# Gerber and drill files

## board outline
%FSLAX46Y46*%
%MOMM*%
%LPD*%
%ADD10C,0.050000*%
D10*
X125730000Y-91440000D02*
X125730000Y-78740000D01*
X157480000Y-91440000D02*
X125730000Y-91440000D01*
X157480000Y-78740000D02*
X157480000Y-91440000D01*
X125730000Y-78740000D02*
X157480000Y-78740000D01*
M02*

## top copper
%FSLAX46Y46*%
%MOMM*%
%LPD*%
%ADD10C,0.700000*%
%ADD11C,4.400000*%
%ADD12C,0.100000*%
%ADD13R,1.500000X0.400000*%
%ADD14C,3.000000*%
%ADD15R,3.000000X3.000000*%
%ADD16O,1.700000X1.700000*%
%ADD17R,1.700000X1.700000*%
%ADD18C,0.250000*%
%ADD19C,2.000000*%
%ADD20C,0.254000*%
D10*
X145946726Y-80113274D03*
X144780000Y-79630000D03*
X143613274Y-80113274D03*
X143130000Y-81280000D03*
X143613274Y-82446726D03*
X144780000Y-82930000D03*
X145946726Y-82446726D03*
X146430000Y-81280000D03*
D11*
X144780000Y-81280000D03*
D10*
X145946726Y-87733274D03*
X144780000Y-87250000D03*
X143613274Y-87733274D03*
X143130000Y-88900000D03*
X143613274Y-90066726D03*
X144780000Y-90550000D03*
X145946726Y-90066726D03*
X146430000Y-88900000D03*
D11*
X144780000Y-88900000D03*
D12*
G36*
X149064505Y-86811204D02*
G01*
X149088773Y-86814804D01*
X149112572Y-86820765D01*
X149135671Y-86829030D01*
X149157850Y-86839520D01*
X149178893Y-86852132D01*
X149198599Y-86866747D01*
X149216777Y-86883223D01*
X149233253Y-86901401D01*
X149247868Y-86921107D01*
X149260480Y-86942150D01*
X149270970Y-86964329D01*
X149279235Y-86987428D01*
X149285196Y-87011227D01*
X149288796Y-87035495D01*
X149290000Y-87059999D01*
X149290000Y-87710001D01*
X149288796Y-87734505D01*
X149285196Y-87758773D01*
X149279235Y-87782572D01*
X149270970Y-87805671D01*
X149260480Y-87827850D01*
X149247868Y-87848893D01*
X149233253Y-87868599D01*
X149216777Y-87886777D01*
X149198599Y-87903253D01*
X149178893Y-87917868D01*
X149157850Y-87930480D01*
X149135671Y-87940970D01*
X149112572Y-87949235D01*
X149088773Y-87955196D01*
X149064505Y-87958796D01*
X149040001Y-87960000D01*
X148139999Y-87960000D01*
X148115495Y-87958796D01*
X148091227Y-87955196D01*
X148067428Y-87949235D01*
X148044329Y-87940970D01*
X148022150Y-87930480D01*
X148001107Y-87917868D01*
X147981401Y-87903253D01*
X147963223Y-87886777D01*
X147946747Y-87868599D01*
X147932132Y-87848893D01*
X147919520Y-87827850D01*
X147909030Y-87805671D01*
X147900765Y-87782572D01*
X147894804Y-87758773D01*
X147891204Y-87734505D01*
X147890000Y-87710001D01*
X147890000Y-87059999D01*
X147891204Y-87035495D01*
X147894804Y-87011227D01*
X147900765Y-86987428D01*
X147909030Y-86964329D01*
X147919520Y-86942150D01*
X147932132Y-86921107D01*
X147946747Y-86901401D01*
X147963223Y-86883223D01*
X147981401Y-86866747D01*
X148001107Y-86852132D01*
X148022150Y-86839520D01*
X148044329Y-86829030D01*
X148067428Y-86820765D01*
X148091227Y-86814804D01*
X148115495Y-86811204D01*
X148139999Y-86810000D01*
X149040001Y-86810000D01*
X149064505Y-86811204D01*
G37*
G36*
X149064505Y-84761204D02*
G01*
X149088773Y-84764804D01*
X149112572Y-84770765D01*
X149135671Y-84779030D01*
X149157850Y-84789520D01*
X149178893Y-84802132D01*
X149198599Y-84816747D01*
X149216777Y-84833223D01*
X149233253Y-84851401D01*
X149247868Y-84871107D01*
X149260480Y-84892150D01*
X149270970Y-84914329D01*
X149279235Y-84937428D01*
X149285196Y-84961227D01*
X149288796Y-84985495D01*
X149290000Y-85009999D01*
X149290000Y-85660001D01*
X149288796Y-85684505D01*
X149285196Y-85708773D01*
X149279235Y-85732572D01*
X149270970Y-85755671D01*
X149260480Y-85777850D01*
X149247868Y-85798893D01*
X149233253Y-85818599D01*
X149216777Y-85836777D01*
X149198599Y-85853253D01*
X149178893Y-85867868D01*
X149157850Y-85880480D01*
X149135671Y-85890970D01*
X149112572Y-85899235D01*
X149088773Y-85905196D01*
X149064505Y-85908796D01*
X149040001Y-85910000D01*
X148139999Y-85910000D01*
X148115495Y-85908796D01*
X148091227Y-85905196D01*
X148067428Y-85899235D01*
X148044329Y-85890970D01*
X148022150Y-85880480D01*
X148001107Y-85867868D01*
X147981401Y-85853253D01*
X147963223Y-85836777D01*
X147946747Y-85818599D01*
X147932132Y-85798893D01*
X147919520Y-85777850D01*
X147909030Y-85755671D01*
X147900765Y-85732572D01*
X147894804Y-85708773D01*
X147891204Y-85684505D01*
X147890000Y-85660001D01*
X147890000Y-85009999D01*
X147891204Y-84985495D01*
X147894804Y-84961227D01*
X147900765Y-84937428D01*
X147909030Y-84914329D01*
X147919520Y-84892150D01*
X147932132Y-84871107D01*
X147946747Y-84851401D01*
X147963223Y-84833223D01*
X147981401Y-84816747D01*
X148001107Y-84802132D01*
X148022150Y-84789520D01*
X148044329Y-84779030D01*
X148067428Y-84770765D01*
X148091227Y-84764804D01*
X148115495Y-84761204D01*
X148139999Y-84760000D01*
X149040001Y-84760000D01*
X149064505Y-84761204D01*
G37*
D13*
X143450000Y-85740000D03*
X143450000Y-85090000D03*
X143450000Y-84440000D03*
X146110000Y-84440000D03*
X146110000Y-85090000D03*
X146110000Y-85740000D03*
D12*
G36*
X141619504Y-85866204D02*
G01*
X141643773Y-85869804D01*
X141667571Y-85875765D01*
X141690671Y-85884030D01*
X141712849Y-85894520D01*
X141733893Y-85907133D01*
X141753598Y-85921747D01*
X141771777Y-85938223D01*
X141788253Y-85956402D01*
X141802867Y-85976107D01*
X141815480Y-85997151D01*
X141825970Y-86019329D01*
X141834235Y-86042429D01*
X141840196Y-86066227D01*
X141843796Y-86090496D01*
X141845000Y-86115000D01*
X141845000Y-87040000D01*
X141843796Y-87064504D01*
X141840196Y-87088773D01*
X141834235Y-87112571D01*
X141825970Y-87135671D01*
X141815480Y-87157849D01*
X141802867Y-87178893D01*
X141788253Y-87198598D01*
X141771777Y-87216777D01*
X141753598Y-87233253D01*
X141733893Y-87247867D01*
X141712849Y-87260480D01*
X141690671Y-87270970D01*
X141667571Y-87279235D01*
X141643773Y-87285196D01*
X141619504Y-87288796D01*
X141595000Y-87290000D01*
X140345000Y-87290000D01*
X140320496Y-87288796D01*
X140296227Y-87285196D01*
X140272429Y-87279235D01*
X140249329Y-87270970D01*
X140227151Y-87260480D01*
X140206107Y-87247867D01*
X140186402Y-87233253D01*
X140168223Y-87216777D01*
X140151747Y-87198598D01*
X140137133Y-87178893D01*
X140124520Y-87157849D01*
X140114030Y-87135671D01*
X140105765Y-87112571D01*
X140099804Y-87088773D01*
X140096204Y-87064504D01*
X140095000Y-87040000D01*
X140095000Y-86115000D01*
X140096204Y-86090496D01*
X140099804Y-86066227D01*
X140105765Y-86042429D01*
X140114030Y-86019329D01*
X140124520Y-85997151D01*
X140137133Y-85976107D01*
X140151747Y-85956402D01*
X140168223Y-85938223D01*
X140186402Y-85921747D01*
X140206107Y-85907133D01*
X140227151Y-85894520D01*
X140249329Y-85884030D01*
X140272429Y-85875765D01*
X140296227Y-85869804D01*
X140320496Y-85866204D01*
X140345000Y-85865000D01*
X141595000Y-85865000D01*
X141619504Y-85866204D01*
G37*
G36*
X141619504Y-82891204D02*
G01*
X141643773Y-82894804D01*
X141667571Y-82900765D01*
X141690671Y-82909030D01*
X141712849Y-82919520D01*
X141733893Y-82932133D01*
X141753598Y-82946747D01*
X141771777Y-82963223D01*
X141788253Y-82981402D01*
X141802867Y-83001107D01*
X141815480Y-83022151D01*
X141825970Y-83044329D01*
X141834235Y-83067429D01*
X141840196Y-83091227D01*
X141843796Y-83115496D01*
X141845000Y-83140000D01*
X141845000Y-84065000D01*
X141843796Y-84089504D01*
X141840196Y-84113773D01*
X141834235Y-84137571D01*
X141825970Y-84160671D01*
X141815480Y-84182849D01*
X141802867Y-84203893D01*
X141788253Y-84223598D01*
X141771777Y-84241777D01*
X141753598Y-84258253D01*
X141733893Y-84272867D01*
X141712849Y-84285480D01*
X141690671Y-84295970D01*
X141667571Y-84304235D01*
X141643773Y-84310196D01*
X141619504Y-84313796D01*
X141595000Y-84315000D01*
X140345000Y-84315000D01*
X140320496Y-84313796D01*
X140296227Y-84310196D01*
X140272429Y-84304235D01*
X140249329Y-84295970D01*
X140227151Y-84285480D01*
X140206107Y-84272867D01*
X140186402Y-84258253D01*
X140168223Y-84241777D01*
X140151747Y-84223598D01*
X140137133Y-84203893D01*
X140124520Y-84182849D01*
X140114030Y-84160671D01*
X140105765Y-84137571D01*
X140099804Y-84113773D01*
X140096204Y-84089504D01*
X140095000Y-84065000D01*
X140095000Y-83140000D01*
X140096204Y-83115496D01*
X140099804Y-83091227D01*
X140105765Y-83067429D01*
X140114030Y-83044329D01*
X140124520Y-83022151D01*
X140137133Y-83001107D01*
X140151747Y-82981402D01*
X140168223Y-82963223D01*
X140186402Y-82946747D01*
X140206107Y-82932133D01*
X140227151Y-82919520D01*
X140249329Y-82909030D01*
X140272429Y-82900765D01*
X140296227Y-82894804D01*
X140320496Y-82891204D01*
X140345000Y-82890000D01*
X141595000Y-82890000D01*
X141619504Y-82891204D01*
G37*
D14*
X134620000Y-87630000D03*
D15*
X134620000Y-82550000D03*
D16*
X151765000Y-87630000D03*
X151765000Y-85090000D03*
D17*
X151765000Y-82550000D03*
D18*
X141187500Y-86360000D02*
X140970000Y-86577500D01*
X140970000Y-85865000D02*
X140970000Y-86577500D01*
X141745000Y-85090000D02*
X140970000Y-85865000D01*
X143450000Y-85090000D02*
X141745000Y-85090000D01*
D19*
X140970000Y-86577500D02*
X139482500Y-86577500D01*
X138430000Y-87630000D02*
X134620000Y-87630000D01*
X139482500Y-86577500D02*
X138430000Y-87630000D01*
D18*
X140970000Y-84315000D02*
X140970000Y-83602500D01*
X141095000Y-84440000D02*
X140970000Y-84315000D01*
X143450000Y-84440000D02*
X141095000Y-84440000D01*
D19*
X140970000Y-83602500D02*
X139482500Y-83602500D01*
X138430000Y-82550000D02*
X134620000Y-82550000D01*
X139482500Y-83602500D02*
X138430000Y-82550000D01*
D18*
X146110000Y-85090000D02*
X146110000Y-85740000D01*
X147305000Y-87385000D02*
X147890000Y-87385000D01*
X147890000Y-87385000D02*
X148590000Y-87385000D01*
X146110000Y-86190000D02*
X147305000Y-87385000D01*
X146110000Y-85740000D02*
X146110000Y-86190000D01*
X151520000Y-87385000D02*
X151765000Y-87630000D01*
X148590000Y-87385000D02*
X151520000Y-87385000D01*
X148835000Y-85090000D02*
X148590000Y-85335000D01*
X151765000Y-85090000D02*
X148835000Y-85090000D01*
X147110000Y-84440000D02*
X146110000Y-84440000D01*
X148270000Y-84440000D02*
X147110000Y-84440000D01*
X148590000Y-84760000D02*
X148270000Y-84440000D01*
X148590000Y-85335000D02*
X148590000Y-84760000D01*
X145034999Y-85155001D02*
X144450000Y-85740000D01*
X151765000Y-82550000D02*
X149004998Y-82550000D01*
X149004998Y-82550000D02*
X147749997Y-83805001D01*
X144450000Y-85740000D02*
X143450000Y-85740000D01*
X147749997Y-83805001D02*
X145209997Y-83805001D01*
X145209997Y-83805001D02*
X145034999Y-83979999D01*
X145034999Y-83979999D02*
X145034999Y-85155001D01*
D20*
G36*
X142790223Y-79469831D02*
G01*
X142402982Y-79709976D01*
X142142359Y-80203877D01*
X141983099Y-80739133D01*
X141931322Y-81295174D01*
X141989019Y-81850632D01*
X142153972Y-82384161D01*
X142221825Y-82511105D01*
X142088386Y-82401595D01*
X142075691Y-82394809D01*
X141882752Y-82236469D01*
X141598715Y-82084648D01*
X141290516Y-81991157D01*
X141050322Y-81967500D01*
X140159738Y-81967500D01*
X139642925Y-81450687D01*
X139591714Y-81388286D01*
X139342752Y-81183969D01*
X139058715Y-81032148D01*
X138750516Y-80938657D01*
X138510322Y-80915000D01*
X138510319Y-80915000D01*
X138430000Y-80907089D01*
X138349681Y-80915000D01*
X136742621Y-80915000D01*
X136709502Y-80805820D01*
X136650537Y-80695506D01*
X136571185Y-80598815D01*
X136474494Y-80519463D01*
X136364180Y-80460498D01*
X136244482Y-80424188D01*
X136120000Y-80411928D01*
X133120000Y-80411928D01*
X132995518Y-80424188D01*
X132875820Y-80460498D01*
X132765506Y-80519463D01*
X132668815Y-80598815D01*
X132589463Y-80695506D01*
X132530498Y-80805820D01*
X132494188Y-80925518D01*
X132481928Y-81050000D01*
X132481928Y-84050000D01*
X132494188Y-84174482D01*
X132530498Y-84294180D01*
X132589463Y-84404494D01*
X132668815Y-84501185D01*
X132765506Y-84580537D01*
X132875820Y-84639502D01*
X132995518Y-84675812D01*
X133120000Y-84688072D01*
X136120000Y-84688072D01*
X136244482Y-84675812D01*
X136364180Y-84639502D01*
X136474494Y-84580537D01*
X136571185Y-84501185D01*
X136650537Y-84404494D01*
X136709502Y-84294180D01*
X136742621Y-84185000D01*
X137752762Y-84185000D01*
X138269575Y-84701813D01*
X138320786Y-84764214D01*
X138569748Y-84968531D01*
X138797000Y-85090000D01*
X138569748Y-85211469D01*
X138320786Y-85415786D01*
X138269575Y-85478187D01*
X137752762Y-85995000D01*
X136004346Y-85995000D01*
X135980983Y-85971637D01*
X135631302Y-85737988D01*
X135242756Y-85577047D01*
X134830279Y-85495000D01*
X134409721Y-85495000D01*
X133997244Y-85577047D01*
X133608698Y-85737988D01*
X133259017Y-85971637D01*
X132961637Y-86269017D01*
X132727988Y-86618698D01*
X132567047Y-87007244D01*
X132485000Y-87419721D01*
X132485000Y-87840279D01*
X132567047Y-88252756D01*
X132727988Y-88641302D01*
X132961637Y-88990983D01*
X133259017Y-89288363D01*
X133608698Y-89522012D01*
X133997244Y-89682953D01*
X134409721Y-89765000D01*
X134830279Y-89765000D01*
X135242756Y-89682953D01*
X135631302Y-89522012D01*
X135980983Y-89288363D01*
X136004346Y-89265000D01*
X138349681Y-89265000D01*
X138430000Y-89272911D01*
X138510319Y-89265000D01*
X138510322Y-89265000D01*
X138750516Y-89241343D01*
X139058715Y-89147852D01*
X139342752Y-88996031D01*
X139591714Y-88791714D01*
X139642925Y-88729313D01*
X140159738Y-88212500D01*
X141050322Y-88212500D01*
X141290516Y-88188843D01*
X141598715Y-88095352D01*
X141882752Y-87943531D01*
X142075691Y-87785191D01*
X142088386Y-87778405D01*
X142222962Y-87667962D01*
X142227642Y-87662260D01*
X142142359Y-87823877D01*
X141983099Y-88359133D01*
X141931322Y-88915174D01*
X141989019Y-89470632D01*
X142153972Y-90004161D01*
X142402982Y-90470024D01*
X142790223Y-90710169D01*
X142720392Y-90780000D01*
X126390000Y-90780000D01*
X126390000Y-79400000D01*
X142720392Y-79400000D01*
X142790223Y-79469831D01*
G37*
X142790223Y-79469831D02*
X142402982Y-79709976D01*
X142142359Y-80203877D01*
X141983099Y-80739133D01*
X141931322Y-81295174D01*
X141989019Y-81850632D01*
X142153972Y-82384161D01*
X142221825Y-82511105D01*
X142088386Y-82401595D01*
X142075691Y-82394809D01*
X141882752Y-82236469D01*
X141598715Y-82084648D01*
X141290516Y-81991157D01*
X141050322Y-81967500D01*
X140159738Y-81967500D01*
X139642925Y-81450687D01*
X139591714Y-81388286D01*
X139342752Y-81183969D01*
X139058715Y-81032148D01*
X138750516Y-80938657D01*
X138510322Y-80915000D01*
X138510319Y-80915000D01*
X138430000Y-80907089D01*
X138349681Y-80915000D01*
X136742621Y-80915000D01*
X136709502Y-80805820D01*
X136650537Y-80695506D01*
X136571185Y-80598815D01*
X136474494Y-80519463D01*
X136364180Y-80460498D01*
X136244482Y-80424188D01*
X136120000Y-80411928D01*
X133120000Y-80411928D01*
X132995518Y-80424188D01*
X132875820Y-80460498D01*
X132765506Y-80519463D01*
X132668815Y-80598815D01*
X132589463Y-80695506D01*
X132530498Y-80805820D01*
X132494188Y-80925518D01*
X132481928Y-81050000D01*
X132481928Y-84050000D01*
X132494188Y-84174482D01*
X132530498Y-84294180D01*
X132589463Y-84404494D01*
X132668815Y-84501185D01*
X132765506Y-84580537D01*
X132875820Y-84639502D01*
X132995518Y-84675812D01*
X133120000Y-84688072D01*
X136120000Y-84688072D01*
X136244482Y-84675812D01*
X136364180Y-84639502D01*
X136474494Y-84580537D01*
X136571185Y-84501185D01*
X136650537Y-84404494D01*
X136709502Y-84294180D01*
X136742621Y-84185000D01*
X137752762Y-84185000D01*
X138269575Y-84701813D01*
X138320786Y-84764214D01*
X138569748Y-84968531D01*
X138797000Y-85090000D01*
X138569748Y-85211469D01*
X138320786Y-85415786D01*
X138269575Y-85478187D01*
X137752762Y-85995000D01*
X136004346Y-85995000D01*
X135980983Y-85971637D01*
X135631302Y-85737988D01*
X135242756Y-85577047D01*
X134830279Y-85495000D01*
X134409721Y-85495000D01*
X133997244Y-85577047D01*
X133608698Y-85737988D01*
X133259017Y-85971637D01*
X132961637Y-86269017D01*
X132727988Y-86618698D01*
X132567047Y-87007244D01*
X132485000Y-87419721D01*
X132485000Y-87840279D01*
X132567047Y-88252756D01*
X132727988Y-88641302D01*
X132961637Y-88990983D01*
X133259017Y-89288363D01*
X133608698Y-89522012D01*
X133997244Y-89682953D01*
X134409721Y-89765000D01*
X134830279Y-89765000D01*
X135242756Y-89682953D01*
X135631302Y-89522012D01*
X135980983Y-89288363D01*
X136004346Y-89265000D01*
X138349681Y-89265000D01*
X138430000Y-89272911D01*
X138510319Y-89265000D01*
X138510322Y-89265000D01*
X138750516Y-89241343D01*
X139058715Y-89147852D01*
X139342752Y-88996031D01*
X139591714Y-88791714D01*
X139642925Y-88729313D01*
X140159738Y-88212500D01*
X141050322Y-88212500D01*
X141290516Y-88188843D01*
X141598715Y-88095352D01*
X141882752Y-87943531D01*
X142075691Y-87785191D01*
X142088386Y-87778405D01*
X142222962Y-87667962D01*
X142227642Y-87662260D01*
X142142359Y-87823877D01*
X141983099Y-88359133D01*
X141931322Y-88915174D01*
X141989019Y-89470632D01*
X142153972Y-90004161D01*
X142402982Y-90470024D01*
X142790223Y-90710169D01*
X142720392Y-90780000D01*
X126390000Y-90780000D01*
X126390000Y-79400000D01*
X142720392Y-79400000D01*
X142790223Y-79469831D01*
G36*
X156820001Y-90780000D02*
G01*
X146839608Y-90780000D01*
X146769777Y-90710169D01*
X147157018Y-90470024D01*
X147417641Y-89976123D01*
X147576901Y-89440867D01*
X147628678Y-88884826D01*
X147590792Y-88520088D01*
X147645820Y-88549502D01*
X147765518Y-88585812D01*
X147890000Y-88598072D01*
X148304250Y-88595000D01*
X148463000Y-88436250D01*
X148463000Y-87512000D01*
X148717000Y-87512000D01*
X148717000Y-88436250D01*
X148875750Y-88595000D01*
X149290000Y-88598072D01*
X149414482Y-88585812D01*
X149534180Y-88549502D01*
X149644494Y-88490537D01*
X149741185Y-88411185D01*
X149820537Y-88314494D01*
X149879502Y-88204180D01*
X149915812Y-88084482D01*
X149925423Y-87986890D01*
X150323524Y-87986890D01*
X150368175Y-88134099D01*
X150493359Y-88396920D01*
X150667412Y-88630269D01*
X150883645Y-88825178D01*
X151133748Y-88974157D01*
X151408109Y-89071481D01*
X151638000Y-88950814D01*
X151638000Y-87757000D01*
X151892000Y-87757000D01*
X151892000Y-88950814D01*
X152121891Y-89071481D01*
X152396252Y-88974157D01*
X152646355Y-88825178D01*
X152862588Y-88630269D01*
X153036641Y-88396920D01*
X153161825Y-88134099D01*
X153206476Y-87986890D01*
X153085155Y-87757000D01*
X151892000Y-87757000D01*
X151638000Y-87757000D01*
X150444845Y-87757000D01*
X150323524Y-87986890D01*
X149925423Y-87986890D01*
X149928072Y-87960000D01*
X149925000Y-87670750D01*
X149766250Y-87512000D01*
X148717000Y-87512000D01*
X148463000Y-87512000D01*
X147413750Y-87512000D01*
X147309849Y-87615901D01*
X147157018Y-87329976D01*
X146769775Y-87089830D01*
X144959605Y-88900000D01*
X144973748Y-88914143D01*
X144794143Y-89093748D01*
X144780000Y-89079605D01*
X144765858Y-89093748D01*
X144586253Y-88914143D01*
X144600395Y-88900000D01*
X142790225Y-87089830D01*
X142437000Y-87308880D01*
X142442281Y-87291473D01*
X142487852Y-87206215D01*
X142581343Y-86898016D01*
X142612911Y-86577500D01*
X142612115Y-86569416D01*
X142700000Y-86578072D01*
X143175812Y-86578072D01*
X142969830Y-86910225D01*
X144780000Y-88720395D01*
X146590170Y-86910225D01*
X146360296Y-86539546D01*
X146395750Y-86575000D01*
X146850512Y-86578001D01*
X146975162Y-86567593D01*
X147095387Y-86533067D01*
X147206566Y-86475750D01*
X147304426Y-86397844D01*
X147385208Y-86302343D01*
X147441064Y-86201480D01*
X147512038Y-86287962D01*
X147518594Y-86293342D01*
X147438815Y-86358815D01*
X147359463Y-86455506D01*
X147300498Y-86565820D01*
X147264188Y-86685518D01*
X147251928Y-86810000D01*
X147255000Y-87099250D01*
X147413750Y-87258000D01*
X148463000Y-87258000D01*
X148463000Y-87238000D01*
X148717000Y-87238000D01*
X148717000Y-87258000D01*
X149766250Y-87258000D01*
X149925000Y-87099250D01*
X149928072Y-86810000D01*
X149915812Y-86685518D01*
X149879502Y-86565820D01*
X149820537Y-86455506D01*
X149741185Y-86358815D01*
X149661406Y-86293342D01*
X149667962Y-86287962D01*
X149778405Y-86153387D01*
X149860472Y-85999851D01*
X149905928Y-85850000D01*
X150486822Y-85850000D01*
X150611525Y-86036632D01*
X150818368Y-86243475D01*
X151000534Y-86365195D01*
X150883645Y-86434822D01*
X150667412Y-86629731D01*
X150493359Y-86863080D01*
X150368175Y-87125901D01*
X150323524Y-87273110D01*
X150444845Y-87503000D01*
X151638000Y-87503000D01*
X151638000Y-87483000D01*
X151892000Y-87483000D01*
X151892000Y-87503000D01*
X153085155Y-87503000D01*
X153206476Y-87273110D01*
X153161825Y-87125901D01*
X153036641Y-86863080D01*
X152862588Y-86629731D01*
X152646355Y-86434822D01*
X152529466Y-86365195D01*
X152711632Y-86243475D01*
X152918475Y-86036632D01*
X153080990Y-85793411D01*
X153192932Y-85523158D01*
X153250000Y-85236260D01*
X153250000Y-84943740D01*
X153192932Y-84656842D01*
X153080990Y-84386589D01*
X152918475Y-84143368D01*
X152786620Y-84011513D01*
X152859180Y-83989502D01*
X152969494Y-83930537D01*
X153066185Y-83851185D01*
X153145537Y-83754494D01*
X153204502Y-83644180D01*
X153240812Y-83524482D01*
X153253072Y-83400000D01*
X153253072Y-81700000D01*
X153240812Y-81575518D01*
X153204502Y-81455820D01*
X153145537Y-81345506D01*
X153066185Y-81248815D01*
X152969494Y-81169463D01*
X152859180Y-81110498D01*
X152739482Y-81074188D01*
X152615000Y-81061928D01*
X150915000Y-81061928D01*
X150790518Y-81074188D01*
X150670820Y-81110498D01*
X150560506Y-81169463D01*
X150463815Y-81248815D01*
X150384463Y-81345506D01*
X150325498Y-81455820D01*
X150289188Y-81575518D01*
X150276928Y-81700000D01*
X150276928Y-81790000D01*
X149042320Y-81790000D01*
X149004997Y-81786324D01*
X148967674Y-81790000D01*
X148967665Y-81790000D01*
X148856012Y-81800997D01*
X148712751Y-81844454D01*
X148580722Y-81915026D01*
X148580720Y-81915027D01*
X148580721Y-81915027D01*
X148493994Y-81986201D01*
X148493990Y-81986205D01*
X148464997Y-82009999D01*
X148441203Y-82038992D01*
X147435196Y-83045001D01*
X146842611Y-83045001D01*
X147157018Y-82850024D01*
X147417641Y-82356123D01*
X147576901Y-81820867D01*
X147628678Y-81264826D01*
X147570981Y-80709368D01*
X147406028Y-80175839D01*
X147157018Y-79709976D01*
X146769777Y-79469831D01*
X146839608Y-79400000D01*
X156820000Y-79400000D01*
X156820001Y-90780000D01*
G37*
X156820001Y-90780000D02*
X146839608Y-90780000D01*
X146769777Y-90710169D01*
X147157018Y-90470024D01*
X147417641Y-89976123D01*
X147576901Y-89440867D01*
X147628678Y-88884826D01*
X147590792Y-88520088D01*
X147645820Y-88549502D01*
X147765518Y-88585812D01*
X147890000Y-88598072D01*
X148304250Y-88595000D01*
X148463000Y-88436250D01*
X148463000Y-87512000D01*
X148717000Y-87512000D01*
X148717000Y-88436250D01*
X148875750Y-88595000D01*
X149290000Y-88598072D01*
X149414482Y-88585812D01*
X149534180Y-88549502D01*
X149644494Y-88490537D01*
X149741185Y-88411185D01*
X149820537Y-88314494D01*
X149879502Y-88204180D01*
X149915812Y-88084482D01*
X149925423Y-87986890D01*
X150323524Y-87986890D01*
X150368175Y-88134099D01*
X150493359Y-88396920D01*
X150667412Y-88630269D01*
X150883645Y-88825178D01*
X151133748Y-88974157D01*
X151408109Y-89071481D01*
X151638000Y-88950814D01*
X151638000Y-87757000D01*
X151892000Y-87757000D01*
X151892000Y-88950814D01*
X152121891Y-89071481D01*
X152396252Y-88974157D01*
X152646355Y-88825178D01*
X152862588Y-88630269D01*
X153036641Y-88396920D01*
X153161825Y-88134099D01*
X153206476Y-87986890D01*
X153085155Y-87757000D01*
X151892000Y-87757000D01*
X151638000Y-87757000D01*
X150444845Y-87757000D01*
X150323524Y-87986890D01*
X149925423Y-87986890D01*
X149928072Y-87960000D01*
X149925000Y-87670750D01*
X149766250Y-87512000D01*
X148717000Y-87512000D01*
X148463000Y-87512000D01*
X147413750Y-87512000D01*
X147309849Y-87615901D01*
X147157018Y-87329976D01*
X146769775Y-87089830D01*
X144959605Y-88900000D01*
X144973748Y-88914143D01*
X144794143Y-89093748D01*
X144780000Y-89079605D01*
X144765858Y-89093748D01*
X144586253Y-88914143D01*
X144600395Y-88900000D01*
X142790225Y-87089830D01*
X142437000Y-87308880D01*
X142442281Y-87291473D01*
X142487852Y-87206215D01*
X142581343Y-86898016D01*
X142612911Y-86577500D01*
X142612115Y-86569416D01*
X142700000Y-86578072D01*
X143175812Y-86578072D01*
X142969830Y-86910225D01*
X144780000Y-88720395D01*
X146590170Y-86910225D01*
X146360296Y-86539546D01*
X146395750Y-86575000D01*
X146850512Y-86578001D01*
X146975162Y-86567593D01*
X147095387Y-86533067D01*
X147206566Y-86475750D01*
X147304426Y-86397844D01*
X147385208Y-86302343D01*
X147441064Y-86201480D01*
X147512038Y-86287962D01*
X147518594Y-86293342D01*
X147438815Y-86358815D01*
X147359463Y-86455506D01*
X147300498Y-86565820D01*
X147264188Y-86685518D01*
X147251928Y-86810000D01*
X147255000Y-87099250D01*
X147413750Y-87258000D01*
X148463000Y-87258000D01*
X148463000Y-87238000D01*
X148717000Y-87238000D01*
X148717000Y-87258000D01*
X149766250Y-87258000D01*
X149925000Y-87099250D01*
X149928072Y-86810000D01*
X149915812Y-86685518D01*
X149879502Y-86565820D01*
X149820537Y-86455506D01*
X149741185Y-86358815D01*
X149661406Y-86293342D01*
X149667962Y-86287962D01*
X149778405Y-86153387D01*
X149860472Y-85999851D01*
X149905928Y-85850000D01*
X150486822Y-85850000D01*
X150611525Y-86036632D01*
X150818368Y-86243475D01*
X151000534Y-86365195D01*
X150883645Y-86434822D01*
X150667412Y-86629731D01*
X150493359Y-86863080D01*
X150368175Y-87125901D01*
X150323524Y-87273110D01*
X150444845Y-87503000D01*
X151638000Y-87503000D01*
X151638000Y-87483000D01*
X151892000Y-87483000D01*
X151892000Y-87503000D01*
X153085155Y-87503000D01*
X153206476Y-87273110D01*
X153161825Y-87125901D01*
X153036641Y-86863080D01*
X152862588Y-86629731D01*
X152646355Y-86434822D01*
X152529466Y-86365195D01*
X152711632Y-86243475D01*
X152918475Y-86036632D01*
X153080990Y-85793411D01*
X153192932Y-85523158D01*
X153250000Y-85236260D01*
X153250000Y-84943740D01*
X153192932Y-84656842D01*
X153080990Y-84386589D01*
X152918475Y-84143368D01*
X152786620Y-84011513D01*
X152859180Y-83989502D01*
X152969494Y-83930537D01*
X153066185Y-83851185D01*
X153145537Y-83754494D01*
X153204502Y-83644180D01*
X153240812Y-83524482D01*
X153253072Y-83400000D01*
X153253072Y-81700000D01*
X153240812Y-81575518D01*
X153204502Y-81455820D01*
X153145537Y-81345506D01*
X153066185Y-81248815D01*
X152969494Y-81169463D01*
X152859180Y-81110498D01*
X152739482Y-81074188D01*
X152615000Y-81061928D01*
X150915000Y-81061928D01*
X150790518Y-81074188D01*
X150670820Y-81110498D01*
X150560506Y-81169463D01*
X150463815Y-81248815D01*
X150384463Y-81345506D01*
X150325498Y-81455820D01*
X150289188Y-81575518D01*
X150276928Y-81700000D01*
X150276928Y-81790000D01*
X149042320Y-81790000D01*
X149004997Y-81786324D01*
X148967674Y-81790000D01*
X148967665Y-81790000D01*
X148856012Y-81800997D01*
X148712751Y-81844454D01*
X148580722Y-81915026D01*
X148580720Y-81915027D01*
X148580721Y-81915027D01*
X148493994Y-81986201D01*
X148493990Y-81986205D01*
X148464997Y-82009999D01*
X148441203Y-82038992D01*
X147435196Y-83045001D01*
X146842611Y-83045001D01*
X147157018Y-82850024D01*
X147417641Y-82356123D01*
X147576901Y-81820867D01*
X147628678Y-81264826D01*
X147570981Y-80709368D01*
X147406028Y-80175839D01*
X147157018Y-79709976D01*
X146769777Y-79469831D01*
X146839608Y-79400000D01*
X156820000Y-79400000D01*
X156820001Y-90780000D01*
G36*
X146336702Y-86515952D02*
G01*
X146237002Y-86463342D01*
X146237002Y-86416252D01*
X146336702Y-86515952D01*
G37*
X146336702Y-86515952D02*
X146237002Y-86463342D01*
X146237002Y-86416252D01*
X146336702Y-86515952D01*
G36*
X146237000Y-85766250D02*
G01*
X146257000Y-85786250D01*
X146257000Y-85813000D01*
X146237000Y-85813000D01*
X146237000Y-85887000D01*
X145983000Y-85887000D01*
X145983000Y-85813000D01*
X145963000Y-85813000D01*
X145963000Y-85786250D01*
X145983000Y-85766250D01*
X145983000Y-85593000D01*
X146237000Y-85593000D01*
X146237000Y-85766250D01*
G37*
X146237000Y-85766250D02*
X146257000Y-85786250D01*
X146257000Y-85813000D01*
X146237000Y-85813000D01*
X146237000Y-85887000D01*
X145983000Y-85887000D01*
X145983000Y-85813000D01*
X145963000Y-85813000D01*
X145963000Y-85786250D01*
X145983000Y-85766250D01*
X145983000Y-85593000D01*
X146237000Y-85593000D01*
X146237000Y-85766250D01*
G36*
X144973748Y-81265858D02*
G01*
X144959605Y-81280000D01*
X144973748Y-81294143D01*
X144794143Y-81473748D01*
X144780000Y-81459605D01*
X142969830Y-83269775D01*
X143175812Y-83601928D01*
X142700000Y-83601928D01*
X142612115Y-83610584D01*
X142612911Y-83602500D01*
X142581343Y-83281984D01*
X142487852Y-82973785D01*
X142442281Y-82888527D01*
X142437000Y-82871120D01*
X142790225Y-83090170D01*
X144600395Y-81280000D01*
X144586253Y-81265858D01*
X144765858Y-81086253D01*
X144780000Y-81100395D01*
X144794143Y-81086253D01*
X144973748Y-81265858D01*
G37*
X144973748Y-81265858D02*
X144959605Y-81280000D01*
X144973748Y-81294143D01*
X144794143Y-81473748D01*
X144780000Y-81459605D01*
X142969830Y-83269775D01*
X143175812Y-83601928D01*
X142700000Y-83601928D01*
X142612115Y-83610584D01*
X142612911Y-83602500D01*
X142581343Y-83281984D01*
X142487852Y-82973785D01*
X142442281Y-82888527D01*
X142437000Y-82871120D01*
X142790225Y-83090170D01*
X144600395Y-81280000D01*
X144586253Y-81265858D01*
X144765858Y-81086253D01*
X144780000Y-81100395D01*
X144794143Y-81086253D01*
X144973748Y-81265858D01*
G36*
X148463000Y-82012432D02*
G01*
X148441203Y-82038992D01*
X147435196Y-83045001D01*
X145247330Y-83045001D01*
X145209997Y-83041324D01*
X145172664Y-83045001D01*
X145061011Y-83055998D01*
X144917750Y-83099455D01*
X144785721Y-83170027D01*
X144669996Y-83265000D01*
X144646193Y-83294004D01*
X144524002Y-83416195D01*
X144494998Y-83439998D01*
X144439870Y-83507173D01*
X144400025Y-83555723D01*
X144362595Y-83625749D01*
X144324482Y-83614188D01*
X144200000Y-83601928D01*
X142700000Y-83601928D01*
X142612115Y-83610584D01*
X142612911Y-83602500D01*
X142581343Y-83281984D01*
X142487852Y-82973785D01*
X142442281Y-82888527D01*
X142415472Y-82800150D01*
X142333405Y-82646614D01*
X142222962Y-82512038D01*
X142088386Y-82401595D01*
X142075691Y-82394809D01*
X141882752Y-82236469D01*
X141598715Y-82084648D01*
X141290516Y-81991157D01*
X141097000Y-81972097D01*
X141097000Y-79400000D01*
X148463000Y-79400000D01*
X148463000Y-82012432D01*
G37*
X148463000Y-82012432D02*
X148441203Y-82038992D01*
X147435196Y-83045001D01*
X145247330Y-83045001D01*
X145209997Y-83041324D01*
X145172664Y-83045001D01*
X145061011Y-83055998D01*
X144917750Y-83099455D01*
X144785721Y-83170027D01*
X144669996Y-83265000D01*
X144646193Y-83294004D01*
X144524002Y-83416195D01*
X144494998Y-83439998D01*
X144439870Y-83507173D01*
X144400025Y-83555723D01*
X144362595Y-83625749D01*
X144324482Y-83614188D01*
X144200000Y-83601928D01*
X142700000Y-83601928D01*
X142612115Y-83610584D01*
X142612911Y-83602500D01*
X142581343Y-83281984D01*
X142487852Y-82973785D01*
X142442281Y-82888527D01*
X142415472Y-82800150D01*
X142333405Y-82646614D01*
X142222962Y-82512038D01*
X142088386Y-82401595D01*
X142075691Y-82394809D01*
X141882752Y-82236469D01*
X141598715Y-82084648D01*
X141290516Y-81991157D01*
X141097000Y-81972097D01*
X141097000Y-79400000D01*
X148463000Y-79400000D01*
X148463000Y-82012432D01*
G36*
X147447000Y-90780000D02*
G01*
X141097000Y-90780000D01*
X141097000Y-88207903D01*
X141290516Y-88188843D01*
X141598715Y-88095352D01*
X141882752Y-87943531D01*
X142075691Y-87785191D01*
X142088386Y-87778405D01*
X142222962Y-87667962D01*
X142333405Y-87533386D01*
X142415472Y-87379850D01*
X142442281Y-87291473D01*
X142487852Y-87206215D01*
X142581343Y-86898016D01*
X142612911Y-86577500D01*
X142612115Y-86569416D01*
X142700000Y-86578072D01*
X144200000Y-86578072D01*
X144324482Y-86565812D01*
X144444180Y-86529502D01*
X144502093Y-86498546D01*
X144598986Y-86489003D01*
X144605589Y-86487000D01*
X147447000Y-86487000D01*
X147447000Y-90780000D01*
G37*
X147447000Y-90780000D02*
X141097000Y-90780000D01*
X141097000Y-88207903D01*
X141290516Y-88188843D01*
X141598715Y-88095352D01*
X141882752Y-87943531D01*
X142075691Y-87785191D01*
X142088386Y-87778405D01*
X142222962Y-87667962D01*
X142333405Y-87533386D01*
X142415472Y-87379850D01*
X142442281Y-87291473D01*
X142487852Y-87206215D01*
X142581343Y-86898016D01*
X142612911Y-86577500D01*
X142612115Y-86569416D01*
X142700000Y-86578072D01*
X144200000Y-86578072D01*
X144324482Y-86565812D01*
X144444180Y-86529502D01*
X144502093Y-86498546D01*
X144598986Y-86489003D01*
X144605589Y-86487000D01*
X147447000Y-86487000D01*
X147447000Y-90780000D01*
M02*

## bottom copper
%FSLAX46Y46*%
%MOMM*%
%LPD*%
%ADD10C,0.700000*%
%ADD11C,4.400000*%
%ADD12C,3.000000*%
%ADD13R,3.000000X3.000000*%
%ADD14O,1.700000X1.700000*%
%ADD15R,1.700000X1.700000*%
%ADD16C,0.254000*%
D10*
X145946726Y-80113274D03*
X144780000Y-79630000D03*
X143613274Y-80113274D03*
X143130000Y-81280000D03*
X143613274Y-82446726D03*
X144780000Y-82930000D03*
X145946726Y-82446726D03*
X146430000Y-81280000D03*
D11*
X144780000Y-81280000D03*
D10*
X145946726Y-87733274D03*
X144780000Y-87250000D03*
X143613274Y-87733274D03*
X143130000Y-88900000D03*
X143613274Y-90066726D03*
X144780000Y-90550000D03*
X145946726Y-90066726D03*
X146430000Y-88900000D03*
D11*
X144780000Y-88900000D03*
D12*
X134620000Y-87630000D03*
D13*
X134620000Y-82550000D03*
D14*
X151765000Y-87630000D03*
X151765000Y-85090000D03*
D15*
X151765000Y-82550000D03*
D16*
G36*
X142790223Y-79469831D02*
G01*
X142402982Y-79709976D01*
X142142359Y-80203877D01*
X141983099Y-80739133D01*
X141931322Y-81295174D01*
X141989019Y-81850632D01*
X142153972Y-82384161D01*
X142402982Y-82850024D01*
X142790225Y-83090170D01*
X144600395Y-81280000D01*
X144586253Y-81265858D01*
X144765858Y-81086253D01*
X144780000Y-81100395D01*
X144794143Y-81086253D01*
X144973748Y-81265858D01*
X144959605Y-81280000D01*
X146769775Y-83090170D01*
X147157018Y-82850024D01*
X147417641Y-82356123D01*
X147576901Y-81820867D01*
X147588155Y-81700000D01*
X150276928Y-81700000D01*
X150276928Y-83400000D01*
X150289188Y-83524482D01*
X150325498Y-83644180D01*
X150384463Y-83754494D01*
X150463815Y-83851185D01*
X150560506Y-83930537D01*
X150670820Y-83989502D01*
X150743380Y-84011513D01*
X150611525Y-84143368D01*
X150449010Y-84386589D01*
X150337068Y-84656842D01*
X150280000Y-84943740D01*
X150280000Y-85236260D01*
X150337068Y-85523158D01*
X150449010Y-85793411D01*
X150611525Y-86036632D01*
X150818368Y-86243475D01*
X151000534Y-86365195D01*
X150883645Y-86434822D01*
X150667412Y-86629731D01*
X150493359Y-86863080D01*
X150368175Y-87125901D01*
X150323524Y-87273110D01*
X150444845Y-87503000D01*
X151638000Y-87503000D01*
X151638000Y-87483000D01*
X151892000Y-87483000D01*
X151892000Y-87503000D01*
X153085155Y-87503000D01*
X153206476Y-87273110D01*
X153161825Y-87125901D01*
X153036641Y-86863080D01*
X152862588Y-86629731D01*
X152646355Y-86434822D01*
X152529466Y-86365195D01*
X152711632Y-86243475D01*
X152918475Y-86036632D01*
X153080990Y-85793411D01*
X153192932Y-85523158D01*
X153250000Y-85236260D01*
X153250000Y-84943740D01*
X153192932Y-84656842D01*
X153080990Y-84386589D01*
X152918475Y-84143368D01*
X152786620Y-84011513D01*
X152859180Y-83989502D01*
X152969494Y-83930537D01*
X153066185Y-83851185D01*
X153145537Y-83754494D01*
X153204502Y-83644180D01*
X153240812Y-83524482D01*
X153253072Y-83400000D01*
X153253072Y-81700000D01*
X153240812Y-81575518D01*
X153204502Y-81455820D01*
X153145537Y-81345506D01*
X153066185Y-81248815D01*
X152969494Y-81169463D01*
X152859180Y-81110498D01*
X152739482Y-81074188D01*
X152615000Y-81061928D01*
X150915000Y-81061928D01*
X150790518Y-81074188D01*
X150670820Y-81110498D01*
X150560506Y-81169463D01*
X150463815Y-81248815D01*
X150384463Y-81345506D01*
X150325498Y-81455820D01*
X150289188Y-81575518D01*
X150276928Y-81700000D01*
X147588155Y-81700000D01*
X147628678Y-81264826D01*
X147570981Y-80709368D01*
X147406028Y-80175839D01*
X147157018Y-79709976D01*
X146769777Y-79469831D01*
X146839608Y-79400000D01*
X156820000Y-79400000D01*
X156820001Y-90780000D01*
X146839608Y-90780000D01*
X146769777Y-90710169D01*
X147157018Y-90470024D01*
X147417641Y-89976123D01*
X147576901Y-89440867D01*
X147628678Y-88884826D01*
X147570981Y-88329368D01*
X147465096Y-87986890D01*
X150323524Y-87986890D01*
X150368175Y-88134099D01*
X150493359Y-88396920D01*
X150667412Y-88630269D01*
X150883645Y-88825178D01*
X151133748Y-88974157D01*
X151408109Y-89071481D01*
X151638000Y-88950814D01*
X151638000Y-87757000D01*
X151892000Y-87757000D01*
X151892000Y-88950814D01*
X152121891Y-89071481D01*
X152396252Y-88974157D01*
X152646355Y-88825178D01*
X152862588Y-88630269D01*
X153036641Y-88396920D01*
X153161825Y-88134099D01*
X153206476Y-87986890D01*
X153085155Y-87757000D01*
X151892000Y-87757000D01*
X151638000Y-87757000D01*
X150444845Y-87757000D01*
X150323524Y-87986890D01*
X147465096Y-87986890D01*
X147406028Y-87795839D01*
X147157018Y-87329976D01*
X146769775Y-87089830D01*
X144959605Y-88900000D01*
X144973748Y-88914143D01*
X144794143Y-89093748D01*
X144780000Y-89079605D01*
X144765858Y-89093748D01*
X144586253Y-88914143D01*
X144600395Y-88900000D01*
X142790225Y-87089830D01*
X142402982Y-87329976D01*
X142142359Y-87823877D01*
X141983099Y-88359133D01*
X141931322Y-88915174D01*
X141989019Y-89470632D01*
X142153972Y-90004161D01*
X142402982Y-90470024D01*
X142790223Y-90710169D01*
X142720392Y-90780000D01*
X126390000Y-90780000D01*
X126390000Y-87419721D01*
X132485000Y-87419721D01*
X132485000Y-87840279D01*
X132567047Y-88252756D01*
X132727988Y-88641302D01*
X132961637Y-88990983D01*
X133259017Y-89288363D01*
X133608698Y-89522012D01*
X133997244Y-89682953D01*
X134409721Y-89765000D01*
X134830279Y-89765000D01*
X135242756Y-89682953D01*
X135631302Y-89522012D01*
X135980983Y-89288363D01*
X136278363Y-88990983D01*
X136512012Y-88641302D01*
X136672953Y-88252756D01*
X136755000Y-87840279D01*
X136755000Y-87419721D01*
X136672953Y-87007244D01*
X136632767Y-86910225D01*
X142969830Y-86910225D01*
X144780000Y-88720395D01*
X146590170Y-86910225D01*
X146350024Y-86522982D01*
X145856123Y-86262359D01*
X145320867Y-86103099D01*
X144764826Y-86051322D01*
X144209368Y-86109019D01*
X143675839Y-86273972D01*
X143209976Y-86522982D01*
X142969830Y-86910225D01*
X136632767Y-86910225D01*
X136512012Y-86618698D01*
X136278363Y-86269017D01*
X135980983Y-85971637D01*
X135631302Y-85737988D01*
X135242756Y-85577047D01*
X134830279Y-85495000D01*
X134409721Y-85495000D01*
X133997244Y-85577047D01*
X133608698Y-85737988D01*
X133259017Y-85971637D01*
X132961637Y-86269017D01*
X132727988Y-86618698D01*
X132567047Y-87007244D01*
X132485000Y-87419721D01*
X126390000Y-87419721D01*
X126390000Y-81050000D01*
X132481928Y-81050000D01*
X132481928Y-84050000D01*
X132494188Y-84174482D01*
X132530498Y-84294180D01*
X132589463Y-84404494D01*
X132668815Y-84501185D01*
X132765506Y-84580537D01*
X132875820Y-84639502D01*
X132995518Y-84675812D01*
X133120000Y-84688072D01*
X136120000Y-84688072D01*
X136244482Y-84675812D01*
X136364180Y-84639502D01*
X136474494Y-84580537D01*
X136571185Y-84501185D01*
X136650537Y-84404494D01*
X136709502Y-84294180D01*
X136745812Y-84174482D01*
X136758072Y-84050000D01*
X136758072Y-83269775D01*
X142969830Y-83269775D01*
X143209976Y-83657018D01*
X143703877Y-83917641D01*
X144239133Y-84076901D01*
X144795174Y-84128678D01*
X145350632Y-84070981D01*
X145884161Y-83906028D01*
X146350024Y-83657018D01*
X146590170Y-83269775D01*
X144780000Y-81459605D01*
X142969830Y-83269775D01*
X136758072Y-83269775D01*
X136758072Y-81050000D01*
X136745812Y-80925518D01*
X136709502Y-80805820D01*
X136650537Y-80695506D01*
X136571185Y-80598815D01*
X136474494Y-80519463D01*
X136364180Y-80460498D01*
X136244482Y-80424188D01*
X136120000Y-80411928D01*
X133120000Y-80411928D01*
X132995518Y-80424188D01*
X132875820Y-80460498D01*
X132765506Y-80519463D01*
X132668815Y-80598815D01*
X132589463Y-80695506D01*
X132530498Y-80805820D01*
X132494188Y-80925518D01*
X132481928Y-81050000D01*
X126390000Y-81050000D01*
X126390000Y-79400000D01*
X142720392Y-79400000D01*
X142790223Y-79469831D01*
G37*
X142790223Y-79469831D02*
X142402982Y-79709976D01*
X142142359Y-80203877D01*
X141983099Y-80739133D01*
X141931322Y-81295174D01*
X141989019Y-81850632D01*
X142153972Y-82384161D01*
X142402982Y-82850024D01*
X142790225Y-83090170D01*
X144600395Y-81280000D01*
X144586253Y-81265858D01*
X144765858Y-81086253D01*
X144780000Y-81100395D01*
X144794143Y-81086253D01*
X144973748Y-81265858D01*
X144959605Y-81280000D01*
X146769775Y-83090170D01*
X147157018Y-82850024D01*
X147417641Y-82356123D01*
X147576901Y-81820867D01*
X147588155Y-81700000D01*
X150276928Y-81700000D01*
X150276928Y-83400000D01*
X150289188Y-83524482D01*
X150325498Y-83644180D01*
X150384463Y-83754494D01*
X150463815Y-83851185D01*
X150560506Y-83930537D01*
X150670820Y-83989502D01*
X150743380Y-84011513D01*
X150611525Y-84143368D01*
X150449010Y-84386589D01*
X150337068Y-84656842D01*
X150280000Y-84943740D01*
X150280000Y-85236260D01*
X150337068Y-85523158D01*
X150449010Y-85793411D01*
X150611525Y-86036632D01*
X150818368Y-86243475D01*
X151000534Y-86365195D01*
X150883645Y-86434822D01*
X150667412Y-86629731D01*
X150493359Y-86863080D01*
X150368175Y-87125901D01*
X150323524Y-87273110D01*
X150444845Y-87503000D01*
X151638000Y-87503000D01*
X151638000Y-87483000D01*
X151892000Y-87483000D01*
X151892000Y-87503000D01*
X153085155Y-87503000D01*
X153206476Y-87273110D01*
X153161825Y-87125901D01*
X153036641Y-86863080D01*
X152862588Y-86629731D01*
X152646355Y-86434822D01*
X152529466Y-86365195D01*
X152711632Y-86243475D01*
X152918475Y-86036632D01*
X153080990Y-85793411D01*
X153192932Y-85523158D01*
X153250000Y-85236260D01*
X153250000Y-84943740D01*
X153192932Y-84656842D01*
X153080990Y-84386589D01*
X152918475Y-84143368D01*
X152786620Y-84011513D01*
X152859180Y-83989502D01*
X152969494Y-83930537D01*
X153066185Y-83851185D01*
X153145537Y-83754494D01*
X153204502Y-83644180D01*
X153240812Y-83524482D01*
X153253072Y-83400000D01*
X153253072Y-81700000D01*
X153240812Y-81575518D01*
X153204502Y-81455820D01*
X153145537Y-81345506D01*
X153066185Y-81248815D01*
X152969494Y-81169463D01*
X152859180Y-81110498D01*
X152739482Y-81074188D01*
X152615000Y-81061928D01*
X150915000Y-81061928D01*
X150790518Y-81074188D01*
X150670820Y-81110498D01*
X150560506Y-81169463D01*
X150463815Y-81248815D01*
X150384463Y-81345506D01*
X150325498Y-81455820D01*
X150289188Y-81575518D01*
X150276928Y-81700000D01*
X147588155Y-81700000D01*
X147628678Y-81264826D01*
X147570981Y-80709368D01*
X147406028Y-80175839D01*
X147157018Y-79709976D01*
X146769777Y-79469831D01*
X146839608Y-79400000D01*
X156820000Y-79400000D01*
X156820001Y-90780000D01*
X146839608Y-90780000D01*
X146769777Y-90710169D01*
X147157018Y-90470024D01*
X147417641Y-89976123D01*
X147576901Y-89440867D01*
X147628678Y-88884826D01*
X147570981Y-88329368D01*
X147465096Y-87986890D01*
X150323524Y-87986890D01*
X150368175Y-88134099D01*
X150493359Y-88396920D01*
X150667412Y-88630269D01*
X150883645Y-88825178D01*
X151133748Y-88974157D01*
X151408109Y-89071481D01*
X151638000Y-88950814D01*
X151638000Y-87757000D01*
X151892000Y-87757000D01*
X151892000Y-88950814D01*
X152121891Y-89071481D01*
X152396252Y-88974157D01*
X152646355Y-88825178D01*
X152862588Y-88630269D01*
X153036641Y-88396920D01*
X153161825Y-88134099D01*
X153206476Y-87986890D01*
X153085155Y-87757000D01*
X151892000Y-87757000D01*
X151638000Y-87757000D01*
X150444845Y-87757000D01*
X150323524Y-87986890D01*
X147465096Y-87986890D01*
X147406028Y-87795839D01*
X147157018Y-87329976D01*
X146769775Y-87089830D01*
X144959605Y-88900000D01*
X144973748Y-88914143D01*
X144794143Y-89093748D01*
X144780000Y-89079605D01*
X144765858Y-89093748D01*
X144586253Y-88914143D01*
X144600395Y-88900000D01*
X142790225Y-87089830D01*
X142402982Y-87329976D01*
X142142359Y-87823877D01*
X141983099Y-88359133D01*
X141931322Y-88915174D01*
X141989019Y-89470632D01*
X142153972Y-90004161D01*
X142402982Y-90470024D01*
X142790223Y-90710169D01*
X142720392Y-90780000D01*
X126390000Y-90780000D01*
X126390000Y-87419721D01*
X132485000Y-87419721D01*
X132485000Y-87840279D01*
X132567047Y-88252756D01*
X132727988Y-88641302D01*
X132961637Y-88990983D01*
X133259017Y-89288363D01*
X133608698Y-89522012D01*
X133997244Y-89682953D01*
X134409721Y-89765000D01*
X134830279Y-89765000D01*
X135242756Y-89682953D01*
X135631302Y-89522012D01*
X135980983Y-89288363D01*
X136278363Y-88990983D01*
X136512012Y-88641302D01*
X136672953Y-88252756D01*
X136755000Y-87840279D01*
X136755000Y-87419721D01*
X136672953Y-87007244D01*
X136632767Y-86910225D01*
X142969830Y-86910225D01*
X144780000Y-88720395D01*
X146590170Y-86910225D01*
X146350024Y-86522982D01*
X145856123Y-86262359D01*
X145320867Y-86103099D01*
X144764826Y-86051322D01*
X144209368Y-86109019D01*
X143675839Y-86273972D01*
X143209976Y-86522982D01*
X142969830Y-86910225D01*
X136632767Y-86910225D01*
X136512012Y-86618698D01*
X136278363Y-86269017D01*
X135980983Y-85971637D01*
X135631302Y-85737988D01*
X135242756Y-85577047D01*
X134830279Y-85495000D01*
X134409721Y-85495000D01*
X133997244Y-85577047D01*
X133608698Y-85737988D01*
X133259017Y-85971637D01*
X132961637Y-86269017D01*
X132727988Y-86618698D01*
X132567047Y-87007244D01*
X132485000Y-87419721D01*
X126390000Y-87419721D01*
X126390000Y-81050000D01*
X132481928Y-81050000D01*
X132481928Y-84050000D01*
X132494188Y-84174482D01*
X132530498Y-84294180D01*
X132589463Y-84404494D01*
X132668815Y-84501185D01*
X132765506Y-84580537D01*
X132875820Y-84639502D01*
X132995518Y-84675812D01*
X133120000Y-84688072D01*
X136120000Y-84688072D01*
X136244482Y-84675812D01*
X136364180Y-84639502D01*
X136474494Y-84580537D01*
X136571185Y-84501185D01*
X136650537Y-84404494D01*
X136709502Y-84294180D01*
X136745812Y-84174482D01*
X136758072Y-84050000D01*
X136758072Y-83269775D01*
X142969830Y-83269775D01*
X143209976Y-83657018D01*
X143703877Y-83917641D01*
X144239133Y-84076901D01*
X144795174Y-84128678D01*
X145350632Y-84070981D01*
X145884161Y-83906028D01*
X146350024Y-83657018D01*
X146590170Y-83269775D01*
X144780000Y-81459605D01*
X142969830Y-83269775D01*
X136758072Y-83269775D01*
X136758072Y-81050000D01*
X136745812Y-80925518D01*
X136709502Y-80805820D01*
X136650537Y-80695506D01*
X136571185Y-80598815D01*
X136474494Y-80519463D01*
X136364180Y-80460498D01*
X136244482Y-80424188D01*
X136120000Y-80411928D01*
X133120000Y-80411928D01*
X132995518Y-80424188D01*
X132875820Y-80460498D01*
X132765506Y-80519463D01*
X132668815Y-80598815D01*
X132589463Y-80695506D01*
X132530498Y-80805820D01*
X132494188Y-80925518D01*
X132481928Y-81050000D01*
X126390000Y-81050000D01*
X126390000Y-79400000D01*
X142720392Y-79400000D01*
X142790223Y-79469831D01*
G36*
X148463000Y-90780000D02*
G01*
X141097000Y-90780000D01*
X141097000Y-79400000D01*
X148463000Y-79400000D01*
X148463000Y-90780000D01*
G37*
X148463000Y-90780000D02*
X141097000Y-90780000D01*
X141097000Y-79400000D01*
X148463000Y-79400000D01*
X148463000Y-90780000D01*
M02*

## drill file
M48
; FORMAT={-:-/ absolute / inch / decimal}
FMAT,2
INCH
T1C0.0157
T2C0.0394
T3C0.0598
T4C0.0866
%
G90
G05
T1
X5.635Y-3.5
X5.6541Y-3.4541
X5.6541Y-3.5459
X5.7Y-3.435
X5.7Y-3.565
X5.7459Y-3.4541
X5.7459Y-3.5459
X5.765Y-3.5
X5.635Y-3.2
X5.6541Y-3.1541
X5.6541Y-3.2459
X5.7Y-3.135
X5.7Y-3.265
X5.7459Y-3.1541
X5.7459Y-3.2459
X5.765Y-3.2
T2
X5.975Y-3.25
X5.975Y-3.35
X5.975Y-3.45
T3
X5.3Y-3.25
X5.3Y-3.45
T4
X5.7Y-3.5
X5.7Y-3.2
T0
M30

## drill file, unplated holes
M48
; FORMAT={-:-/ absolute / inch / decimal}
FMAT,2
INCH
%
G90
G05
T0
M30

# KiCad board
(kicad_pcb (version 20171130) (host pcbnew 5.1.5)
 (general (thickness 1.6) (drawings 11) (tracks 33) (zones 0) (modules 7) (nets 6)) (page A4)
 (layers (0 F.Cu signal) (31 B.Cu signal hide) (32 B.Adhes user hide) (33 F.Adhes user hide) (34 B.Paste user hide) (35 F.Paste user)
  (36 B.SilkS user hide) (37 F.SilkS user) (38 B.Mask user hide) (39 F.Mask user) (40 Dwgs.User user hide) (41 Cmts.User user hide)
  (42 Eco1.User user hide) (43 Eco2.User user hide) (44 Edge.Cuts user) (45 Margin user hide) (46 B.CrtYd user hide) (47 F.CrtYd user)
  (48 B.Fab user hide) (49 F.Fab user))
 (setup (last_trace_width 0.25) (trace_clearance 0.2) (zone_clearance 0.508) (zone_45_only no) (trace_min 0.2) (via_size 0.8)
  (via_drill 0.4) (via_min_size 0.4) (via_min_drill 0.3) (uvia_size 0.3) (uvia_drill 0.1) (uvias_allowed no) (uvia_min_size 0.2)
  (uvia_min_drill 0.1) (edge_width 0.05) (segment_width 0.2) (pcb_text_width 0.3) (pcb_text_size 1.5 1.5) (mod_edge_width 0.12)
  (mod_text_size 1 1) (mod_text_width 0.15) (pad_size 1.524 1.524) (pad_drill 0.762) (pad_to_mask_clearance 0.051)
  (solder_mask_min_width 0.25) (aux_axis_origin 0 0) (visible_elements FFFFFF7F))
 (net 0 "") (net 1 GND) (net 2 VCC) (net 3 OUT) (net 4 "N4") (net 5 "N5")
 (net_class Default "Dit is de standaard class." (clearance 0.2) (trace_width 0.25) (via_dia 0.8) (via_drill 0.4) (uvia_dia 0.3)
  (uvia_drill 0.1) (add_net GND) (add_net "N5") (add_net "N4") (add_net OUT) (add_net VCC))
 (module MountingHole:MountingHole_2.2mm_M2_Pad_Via (layer F.Cu) (at 144.78 81.28)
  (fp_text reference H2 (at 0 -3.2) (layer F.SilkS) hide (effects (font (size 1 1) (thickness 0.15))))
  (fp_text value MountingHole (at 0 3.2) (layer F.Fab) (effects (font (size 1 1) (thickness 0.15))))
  (pad 1 thru_hole circle (at 1.166726 -1.166726) (size 0.7 0.7) (drill 0.4) (layers *.Cu *.Mask) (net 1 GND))
  (pad 1 thru_hole circle (at 0 -1.65) (size 0.7 0.7) (drill 0.4) (layers *.Cu *.Mask) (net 1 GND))
  (pad 1 thru_hole circle (at -1.166726 -1.166726) (size 0.7 0.7) (drill 0.4) (layers *.Cu *.Mask) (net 1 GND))
  (pad 1 thru_hole circle (at -1.65 0) (size 0.7 0.7) (drill 0.4) (layers *.Cu *.Mask) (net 1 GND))
  (pad 1 thru_hole circle (at -1.166726 1.166726) (size 0.7 0.7) (drill 0.4) (layers *.Cu *.Mask) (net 1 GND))
  (pad 1 thru_hole circle (at 0 1.65) (size 0.7 0.7) (drill 0.4) (layers *.Cu *.Mask) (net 1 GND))
  (pad 1 thru_hole circle (at 1.166726 1.166726) (size 0.7 0.7) (drill 0.4) (layers *.Cu *.Mask) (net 1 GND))
  (pad 1 thru_hole circle (at 1.65 0) (size 0.7 0.7) (drill 0.4) (layers *.Cu *.Mask) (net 1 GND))
  (pad 1 thru_hole circle (at 0 0) (size 4.4 4.4) (drill 2.2) (layers *.Cu *.Mask) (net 1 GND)))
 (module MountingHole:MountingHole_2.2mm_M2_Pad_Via (layer F.Cu) (at 144.78 88.9)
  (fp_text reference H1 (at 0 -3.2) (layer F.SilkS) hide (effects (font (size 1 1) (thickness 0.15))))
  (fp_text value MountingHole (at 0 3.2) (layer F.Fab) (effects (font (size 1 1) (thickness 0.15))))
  (pad 1 thru_hole circle (at 1.166726 -1.166726) (size 0.7 0.7) (drill 0.4) (layers *.Cu *.Mask) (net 1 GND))
  (pad 1 thru_hole circle (at 0 -1.65) (size 0.7 0.7) (drill 0.4) (layers *.Cu *.Mask) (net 1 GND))
  (pad 1 thru_hole circle (at -1.166726 -1.166726) (size 0.7 0.7) (drill 0.4) (layers *.Cu *.Mask) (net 1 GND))
  (pad 1 thru_hole circle (at -1.65 0) (size 0.7 0.7) (drill 0.4) (layers *.Cu *.Mask) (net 1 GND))
  (pad 1 thru_hole circle (at -1.166726 1.166726) (size 0.7 0.7) (drill 0.4) (layers *.Cu *.Mask) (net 1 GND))
  (pad 1 thru_hole circle (at 0 1.65) (size 0.7 0.7) (drill 0.4) (layers *.Cu *.Mask) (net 1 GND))
  (pad 1 thru_hole circle (at 1.166726 1.166726) (size 0.7 0.7) (drill 0.4) (layers *.Cu *.Mask) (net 1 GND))
  (pad 1 thru_hole circle (at 1.65 0) (size 0.7 0.7) (drill 0.4) (layers *.Cu *.Mask) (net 1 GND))
  (pad 1 thru_hole circle (at 0 0) (size 4.4 4.4) (drill 2.2) (layers *.Cu *.Mask) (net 1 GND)))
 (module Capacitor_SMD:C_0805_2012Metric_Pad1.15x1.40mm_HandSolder (layer F.Cu) (at 148.59 86.36 270)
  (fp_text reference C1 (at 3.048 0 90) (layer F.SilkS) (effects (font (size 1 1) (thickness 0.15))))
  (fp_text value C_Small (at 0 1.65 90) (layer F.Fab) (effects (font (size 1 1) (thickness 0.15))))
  (pad 2 smd roundrect (at 1.025 0 270) (size 1.15 1.4) (layers F.Cu F.Paste F.Mask) (roundrect_rratio 0.217391) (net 1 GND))
  (pad 1 smd roundrect (at -1.025 0 270) (size 1.15 1.4) (layers F.Cu F.Paste F.Mask) (roundrect_rratio 0.217391) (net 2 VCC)))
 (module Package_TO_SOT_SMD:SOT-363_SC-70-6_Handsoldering (layer F.Cu) (at 144.78 85.09 180)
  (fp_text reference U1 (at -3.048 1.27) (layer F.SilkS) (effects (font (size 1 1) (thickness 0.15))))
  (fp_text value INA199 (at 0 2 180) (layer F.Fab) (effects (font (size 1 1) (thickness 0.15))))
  (pad 6 smd rect (at 1.33 -0.65 180) (size 1.5 0.4) (layers F.Cu F.Paste F.Mask) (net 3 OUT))
  (pad 5 smd rect (at 1.33 0 180) (size 1.5 0.4) (layers F.Cu F.Paste F.Mask) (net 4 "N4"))
  (pad 4 smd rect (at 1.33 0.65 180) (size 1.5 0.4) (layers F.Cu F.Paste F.Mask) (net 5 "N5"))
  (pad 3 smd rect (at -1.33 0.65 180) (size 1.5 0.4) (layers F.Cu F.Paste F.Mask) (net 2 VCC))
  (pad 2 smd rect (at -1.33 0 180) (size 1.5 0.4) (layers F.Cu F.Paste F.Mask) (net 1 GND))
  (pad 1 smd rect (at -1.33 -0.65 180) (size 1.5 0.4) (layers F.Cu F.Paste F.Mask) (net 1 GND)))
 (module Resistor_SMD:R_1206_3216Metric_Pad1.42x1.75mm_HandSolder (layer F.Cu) (at 140.97 85.09 270)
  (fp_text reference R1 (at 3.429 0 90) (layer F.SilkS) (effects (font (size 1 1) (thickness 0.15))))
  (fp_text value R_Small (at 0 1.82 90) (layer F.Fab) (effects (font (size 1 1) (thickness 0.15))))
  (pad 2 smd roundrect (at 1.4875 0 270) (size 1.425 1.75) (layers F.Cu F.Paste F.Mask) (roundrect_rratio 0.175439) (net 4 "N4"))
  (pad 1 smd roundrect (at -1.4875 0 270) (size 1.425 1.75) (layers F.Cu F.Paste F.Mask) (roundrect_rratio 0.175439) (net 5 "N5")))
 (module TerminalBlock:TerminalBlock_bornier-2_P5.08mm (layer F.Cu) (at 134.62 82.55 270)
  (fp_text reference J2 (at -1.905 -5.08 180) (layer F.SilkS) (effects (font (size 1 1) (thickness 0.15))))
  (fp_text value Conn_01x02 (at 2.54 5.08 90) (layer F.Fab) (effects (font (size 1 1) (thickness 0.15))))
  (pad 2 thru_hole circle (at 5.08 0 270) (size 3 3) (drill 1.52) (layers *.Cu *.Mask) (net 4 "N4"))
  (pad 1 thru_hole rect (at 0 0 270) (size 3 3) (drill 1.52) (layers *.Cu *.Mask) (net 5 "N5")))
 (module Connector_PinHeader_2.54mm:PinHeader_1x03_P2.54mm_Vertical (layer F.Cu) (at 151.765 82.55)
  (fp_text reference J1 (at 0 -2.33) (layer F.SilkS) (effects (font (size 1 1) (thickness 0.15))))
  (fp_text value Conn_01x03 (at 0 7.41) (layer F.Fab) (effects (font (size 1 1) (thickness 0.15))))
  (pad 3 thru_hole oval (at 0 5.08) (size 1.7 1.7) (drill 1) (layers *.Cu *.Mask) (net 1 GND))
  (pad 2 thru_hole oval (at 0 2.54) (size 1.7 1.7) (drill 1) (layers *.Cu *.Mask) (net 2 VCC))
  (pad 1 thru_hole rect (at 0 0) (size 1.7 1.7) (drill 1) (layers *.Cu *.Mask) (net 3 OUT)))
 (gr_line (start 125.73 91.44) (end 125.73 78.74) (layer Edge.Cuts) (width 0.05))
 (gr_line (start 157.48 91.44) (end 125.73 91.44) (layer Edge.Cuts) (width 0.05))
 (gr_line (start 157.48 78.74) (end 157.48 91.44) (layer Edge.Cuts) (width 0.05))
 (gr_line (start 125.73 78.74) (end 157.48 78.74) (layer Edge.Cuts) (width 0.05))
 (segment (start 141.1875 86.36) (end 140.97 86.5775) (width 0.25) (layer F.Cu) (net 4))
 (segment (start 140.97 85.865) (end 140.97 86.5775) (width 0.25) (layer F.Cu) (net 4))
 (segment (start 141.745 85.09) (end 140.97 85.865) (width 0.25) (layer F.Cu) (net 4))
 (segment (start 143.45 85.09) (end 141.745 85.09) (width 0.25) (layer F.Cu) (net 4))
 (segment (start 140.97 86.5775) (end 139.4825 86.5775) (width 2) (layer F.Cu) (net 4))
 (segment (start 138.43 87.63) (end 134.62 87.63) (width 2) (layer F.Cu) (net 4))
 (segment (start 139.4825 86.5775) (end 138.43 87.63) (width 2) (layer F.Cu) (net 4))
 (segment (start 140.97 84.315) (end 140.97 83.6025) (width 0.25) (layer F.Cu) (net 5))
 (segment (start 141.095 84.44) (end 140.97 84.315) (width 0.25) (layer F.Cu) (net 5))
 (segment (start 143.45 84.44) (end 141.095 84.44) (width 0.25) (layer F.Cu) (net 5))
 (segment (start 140.97 83.6025) (end 139.4825 83.6025) (width 2) (layer F.Cu) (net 5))
 (segment (start 138.43 82.55) (end 134.62 82.55) (width 2) (layer F.Cu) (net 5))
 (segment (start 139.4825 83.6025) (end 138.43 82.55) (width 2) (layer F.Cu) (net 5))
 (segment (start 146.11 85.09) (end 146.11 85.74) (width 0.25) (layer F.Cu) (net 1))
 (segment (start 147.305 87.385) (end 147.89 87.385) (width 0.25) (layer F.Cu) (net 1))
 (segment (start 147.89 87.385) (end 148.59 87.385) (width 0.25) (layer F.Cu) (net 1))
 (segment (start 146.11 86.19) (end 147.305 87.385) (width 0.25) (layer F.Cu) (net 1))
 (segment (start 146.11 85.74) (end 146.11 86.19) (width 0.25) (layer F.Cu) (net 1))
 (segment (start 151.52 87.385) (end 151.765 87.63) (width 0.25) (layer F.Cu) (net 1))
 (segment (start 148.59 87.385) (end 151.52 87.385) (width 0.25) (layer F.Cu) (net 1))
 (segment (start 148.835 85.09) (end 148.59 85.335) (width 0.25) (layer F.Cu) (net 2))
 (segment (start 151.765 85.09) (end 148.835 85.09) (width 0.25) (layer F.Cu) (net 2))
 (segment (start 147.11 84.44) (end 146.11 84.44) (width 0.25) (layer F.Cu) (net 2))
 (segment (start 148.27 84.44) (end 147.11 84.44) (width 0.25) (layer F.Cu) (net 2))
 (segment (start 148.59 84.76) (end 148.27 84.44) (width 0.25) (layer F.Cu) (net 2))
 (segment (start 148.59 85.335) (end 148.59 84.76) (width 0.25) (layer F.Cu) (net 2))
 (segment (start 145.034999 85.155001) (end 144.45 85.74) (width 0.25) (layer F.Cu) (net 3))
 (segment (start 151.765 82.55) (end 149.004998 82.55) (width 0.25) (layer F.Cu) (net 3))
 (segment (start 149.004998 82.55) (end 147.749997 83.805001) (width 0.25) (layer F.Cu) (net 3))
 (segment (start 144.45 85.74) (end 143.45 85.74) (width 0.25) (layer F.Cu) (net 3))
 (segment (start 147.749997 83.805001) (end 145.209997 83.805001) (width 0.25) (layer F.Cu) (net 3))
 (segment (start 145.209997 83.805001) (end 145.034999 83.979999) (width 0.25) (layer F.Cu) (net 3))
 (segment (start 145.034999 83.979999) (end 145.034999 85.155001) (width 0.25) (layer F.Cu) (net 3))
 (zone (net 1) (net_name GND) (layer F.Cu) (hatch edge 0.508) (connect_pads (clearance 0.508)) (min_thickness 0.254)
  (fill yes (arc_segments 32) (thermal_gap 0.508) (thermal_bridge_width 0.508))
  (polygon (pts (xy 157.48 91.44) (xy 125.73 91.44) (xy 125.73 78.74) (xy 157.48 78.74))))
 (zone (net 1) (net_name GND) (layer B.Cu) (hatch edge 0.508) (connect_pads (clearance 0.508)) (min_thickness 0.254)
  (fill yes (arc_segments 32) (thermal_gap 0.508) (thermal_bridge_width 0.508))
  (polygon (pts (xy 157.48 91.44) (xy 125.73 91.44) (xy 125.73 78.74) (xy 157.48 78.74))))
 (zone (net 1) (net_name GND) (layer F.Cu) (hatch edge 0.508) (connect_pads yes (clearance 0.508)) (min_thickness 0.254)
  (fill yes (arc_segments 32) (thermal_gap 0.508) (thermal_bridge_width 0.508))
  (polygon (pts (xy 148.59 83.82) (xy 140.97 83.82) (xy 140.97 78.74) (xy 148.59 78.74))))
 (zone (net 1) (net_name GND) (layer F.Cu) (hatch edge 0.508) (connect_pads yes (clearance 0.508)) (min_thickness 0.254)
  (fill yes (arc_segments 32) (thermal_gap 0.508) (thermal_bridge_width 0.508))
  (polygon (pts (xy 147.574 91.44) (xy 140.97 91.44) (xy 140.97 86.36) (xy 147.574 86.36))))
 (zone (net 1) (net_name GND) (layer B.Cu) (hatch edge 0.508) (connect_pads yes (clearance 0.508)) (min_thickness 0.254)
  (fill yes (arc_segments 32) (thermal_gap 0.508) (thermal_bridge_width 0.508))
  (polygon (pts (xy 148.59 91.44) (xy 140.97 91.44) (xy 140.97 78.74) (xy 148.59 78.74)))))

